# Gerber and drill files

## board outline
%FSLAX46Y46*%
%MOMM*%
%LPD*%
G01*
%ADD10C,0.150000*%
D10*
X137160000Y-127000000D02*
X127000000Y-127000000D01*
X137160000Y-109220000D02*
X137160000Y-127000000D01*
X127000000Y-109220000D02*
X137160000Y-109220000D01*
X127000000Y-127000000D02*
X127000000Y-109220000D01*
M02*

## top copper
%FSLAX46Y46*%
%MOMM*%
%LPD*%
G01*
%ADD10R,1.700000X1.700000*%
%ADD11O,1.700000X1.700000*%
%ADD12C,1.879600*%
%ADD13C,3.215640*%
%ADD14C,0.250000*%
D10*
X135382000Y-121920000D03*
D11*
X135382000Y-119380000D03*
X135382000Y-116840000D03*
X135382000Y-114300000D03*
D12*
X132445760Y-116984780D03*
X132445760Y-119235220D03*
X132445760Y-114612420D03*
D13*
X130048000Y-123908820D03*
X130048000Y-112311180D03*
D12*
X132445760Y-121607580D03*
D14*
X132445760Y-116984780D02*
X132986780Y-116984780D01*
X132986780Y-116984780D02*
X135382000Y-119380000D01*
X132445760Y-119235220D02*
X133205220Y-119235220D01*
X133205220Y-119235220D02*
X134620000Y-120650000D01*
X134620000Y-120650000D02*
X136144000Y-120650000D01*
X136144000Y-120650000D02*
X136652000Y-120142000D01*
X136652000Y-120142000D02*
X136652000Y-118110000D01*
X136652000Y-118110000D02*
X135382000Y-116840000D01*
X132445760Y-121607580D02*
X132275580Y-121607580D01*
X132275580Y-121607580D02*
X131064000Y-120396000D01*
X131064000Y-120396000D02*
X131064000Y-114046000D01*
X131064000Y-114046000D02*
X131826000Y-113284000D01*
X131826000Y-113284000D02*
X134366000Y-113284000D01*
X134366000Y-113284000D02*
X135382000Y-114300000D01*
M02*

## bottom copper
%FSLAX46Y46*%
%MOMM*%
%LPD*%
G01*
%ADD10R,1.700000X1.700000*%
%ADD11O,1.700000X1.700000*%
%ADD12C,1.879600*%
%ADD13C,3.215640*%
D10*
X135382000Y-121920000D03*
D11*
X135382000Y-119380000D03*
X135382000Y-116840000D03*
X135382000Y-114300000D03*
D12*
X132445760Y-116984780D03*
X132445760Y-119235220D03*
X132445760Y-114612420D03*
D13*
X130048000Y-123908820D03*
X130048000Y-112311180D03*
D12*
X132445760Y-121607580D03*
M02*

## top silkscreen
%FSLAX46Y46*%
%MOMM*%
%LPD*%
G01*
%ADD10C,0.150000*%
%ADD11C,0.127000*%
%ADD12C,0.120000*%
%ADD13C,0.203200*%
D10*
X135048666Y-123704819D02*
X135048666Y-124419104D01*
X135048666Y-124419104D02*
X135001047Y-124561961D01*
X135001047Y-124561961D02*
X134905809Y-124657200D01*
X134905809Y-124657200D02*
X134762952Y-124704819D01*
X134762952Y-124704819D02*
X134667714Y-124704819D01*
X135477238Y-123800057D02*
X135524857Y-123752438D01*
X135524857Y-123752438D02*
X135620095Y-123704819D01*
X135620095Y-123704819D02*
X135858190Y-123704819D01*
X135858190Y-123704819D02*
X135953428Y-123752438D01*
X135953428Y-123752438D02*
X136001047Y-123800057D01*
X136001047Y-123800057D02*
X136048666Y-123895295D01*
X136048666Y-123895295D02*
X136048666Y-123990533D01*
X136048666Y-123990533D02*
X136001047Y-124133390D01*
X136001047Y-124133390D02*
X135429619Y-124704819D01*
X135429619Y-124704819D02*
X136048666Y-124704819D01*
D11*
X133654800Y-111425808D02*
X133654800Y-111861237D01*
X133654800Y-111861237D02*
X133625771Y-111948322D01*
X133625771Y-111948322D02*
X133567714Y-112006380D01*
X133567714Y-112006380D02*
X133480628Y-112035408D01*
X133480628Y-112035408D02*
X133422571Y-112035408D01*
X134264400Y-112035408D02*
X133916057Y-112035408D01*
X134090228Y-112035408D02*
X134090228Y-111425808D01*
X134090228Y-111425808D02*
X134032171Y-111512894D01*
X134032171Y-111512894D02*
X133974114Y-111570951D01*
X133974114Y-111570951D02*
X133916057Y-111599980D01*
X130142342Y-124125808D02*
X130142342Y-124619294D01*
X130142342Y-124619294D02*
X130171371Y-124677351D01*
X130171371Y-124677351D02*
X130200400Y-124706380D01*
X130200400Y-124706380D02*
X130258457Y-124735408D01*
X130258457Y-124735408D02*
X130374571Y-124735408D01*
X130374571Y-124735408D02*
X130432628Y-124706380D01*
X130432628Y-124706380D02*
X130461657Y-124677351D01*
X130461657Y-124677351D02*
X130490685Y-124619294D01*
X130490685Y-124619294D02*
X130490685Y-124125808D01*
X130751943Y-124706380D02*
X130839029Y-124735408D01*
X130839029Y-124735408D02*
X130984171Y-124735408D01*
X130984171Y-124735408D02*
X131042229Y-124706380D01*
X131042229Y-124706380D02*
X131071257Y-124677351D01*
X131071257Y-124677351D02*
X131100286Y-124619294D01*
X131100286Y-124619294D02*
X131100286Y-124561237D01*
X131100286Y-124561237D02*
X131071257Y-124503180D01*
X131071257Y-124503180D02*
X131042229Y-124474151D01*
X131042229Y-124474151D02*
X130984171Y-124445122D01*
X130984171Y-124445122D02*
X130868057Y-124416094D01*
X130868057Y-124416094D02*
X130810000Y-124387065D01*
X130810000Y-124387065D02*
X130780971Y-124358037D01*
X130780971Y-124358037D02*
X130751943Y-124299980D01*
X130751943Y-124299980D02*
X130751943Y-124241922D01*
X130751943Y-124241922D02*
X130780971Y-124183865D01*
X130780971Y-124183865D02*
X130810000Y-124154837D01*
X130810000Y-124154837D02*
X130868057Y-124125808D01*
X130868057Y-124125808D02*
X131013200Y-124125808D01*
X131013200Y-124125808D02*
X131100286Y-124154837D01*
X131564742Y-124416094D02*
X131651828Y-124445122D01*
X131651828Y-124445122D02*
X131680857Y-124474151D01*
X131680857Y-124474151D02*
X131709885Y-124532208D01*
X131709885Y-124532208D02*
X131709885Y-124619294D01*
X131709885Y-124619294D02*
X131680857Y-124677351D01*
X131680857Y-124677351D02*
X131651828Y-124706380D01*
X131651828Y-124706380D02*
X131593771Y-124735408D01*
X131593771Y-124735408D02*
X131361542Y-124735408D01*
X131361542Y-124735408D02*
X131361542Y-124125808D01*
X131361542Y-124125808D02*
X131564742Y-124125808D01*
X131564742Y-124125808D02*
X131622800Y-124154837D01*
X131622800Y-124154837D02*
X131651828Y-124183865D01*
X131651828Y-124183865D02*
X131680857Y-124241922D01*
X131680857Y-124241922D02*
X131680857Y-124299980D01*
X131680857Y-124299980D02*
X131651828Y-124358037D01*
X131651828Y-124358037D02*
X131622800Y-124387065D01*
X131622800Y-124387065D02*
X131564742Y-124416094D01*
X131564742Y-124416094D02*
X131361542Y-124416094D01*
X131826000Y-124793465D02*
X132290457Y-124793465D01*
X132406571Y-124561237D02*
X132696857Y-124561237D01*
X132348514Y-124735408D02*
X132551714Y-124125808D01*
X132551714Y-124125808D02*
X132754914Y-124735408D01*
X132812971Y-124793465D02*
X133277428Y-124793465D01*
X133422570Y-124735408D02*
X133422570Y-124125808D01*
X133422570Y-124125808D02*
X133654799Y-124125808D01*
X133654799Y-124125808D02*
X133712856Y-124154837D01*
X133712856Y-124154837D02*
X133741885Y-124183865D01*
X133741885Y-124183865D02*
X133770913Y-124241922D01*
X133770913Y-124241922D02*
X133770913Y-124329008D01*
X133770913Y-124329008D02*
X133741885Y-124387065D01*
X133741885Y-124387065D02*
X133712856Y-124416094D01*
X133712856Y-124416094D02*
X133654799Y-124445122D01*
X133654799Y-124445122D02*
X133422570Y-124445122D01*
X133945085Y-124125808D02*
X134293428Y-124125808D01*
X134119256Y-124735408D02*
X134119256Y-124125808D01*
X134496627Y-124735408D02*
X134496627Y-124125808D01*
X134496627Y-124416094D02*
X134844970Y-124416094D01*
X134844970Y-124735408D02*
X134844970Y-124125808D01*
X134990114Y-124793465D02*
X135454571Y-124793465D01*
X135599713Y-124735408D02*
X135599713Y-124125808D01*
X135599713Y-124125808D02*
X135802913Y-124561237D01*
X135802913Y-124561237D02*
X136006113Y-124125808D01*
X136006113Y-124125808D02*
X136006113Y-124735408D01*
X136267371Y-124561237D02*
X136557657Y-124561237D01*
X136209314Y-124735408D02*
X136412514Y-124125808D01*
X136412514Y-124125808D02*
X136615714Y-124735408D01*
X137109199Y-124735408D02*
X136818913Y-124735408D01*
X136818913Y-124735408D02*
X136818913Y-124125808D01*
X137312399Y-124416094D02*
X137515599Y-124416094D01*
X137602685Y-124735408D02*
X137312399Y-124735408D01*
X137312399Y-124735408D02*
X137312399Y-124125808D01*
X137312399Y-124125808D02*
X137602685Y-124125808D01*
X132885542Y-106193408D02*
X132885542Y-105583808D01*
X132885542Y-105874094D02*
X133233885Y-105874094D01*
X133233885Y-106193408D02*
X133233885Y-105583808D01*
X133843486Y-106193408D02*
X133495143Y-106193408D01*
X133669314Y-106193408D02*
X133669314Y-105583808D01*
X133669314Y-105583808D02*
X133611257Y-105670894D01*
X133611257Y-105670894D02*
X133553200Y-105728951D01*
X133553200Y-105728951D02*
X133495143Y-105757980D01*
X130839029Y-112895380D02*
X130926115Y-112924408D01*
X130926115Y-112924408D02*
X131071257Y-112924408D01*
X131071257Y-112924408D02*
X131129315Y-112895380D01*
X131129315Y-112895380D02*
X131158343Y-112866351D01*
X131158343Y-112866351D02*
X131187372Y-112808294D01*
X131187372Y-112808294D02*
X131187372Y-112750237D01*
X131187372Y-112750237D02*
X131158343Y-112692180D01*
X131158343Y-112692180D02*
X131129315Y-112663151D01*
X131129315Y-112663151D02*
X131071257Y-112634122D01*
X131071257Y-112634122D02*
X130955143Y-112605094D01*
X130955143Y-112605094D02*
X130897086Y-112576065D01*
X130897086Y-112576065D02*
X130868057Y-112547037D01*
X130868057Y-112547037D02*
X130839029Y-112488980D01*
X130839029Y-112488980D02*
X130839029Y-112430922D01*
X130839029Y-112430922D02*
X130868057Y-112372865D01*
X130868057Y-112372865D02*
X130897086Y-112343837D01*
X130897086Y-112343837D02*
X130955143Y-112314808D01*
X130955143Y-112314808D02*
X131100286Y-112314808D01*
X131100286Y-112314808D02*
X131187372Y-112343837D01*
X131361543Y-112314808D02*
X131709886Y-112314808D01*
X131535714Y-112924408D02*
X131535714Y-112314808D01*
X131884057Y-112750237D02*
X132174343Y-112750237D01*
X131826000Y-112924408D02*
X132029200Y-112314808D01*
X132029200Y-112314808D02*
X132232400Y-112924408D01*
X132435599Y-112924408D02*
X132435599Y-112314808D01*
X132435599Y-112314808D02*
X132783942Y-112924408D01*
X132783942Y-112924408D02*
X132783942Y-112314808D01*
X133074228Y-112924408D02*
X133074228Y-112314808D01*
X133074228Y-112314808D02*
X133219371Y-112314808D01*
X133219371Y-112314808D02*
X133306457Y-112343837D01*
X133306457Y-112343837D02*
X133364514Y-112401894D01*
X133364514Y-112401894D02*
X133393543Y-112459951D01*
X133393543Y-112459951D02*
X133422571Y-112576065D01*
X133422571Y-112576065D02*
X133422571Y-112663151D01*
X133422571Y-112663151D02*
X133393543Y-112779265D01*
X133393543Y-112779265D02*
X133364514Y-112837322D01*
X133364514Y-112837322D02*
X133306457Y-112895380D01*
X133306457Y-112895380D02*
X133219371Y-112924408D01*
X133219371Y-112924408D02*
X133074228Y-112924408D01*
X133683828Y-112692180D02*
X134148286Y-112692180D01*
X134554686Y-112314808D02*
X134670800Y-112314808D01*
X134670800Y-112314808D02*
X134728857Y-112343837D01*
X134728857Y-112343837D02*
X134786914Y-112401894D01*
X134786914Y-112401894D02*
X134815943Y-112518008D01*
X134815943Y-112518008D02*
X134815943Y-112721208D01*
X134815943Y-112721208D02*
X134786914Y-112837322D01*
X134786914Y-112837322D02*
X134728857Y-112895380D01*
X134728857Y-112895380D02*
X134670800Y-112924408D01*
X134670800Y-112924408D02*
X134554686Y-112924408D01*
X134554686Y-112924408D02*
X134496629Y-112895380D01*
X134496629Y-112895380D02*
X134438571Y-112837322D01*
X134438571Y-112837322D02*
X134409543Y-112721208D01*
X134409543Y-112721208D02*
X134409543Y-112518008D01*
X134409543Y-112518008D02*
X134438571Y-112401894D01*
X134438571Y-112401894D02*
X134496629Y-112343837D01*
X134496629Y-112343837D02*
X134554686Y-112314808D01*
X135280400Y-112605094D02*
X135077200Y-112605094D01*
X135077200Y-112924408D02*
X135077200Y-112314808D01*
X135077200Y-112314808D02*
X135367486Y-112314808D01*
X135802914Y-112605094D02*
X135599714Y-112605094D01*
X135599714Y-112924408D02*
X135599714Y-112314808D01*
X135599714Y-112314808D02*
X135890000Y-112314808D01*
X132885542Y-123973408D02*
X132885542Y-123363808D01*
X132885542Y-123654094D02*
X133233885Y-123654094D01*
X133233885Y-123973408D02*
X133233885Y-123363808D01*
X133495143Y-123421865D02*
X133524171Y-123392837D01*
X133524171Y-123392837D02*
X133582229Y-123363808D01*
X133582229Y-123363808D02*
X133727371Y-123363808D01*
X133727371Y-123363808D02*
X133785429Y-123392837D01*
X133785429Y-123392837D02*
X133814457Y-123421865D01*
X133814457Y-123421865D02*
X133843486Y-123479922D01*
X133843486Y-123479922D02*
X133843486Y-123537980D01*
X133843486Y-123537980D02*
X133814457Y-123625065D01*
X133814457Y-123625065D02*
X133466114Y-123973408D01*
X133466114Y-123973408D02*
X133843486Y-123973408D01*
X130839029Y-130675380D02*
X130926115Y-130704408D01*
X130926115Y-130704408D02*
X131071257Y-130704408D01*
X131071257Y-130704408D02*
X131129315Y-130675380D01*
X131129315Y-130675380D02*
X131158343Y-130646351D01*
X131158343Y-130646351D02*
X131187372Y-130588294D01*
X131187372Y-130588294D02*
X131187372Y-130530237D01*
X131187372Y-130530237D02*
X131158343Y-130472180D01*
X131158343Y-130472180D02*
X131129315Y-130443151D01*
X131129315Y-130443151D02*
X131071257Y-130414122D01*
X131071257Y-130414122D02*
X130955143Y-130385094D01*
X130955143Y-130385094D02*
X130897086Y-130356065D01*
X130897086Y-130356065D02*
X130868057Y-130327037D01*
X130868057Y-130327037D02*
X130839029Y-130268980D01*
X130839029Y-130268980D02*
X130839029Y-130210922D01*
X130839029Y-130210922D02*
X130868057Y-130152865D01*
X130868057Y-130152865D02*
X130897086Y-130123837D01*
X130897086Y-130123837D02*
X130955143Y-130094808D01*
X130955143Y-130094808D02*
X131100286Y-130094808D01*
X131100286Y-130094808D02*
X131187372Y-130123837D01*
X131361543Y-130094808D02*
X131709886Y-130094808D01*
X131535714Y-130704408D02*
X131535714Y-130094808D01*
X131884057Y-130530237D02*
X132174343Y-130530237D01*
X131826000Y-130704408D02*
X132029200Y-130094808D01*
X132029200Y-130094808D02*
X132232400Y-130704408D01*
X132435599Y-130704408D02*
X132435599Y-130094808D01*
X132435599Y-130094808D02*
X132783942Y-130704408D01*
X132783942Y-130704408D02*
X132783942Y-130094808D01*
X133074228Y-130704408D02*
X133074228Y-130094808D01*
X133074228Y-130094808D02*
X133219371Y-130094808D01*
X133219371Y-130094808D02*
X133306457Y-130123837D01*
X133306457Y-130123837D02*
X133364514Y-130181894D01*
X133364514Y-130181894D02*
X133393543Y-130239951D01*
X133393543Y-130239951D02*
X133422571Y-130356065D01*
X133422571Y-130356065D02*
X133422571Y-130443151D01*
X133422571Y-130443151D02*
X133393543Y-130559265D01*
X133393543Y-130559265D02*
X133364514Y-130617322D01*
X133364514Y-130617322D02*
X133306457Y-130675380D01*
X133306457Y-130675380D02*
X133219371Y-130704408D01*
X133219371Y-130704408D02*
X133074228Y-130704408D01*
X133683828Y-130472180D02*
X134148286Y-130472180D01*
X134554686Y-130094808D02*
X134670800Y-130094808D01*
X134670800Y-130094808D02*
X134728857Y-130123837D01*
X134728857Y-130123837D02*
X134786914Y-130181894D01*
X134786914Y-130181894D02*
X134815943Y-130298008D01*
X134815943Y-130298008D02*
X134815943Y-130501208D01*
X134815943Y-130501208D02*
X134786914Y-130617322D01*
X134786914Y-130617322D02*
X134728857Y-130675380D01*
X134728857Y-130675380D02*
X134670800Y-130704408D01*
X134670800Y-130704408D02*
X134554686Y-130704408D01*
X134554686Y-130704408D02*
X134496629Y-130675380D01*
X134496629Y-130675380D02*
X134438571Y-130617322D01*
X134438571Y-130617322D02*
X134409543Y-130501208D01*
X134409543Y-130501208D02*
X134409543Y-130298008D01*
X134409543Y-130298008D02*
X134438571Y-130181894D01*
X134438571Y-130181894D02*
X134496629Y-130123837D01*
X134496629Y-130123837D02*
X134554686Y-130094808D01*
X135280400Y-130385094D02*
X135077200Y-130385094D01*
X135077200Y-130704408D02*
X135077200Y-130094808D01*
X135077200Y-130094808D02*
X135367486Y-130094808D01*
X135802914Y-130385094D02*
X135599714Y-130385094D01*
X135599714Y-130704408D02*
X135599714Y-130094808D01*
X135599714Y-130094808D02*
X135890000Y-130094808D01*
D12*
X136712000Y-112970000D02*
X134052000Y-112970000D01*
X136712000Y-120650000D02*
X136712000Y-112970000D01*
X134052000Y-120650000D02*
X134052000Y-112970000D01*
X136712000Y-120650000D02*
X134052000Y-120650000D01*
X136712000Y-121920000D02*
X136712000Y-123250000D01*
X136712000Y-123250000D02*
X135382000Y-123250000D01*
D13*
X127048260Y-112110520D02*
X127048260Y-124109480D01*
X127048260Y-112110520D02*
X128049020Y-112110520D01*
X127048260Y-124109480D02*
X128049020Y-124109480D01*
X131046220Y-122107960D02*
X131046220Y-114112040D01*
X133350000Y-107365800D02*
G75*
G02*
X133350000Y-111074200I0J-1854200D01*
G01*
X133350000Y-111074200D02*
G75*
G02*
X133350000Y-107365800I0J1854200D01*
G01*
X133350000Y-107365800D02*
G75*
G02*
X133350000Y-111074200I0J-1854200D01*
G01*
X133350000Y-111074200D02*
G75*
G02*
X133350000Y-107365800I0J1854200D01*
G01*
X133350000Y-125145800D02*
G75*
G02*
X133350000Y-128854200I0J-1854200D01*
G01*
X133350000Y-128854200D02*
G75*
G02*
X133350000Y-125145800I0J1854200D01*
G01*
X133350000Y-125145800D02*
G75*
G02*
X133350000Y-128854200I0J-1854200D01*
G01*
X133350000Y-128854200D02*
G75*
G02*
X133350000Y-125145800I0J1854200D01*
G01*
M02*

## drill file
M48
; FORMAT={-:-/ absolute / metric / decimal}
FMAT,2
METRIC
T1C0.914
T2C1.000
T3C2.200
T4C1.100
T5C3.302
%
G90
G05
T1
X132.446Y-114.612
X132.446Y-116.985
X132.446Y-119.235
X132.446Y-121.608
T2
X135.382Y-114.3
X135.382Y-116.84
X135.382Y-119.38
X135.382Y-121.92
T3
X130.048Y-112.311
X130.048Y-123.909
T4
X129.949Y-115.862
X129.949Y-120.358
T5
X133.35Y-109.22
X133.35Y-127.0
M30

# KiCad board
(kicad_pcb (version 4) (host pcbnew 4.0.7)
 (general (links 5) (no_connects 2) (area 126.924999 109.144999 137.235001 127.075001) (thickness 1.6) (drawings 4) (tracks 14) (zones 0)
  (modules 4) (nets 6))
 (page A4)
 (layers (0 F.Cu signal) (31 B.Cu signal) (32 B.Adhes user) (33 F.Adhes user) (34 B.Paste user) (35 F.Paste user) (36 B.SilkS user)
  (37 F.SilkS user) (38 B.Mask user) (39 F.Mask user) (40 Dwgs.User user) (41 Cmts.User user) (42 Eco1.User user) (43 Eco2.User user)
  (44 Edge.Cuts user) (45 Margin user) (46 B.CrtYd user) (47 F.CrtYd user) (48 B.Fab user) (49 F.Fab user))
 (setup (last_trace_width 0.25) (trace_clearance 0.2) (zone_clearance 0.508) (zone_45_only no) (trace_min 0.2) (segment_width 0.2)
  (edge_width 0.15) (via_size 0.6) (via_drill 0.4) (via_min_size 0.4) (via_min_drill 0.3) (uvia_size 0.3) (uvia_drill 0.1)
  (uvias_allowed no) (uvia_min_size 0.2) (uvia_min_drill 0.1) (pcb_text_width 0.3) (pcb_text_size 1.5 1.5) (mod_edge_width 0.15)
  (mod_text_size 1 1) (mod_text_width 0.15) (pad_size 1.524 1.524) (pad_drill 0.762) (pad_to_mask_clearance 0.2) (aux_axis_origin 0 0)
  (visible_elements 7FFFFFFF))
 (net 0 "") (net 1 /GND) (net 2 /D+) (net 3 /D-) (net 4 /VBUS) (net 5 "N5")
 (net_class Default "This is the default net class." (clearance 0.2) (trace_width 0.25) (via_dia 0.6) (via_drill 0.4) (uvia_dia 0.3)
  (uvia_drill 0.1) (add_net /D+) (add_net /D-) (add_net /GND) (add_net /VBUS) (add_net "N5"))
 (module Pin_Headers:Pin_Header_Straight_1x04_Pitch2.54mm (layer F.Cu) (at 135.382 121.92 180)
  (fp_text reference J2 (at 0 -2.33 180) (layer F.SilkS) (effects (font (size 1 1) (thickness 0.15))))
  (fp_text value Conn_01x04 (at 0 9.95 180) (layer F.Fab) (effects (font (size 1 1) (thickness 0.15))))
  (fp_line (start -1.33 8.95) (end 1.33 8.95) (layer F.SilkS) (width 0.12))
  (fp_line (start -1.33 1.27) (end -1.33 8.95) (layer F.SilkS) (width 0.12))
  (fp_line (start 1.33 1.27) (end 1.33 8.95) (layer F.SilkS) (width 0.12))
  (fp_line (start -1.33 1.27) (end 1.33 1.27) (layer F.SilkS) (width 0.12))
  (fp_line (start -1.33 0) (end -1.33 -1.33) (layer F.SilkS) (width 0.12))
  (fp_line (start -1.33 -1.33) (end 0 -1.33) (layer F.SilkS) (width 0.12))
  (pad 1 thru_hole rect (at 0 0 180) (size 1.7 1.7) (drill 1) (layers *.Cu *.Mask) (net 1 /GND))
  (pad 2 thru_hole oval (at 0 2.54 180) (size 1.7 1.7) (drill 1) (layers *.Cu *.Mask) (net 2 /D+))
  (pad 3 thru_hole oval (at 0 5.08 180) (size 1.7 1.7) (drill 1) (layers *.Cu *.Mask) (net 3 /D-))
  (pad 4 thru_hole oval (at 0 7.62 180) (size 1.7 1.7) (drill 1) (layers *.Cu *.Mask) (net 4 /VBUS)))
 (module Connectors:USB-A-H (layer F.Cu) (at 130.048 118.11)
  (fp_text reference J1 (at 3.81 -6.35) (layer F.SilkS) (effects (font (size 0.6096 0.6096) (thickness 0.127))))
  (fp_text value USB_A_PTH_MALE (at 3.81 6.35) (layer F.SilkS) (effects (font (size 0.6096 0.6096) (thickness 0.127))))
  (fp_line (start -2.99974 -5.99948) (end -2.99974 5.99948) (layer F.SilkS) (width 0.2032))
  (fp_line (start -2.99974 -5.99948) (end -1.99898 -5.99948) (layer F.SilkS) (width 0.2032))
  (fp_line (start -2.99974 5.99948) (end -1.99898 5.99948) (layer F.SilkS) (width 0.2032))
  (fp_line (start 0.99822 3.99796) (end 0.99822 -3.99796) (layer F.SilkS) (width 0.2032))
  (pad D+ thru_hole circle (at 2.39776 -1.12522) (size 1.8796 1.8796) (drill 0.9144) (layers *.Cu *.Mask) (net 2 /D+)
   (solder_mask_margin 0.1016))
  (pad D- thru_hole circle (at 2.39776 1.12522) (size 1.8796 1.8796) (drill 0.9144) (layers *.Cu *.Mask) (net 3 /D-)
   (solder_mask_margin 0.1016))
  (pad GND thru_hole circle (at 2.39776 -3.49758) (size 1.8796 1.8796) (drill 0.9144) (layers *.Cu *.Mask) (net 1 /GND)
   (solder_mask_margin 0.1016))
  (pad SHLD thru_hole circle (at 0 5.79882) (size 3.21564 3.21564) (drill 2.19964) (layers *.Cu *.Mask) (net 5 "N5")
   (solder_mask_margin 0.1016))
  (pad SHLD thru_hole circle (at 0 -5.79882) (size 3.21564 3.21564) (drill 2.19964) (layers *.Cu *.Mask) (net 5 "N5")
   (solder_mask_margin 0.1016))
  (pad VBUS thru_hole circle (at 2.39776 3.49758) (size 1.8796 1.8796) (drill 0.9144) (layers *.Cu *.Mask) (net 4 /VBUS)
   (solder_mask_margin 0.1016))
  (pad "" np_thru_hole circle (at -0.09906 -2.2479) (size 1.09982 1.09982) (drill 1.09982) (layers *.Cu *.Mask) (solder_mask_margin 0.1016))
  (pad "" np_thru_hole circle (at -0.09906 2.2479) (size 1.09982 1.09982) (drill 1.09982) (layers *.Cu *.Mask) (solder_mask_margin 0.1016)))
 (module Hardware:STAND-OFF (layer F.Cu) (at 133.35 109.22)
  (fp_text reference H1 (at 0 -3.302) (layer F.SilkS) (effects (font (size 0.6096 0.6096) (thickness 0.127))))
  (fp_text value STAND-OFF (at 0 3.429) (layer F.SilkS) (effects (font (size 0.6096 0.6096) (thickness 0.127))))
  (fp_arc (start 0 0) (end 0 -1.8542) (angle 180) (layer F.SilkS) (width 0.2032))
  (fp_arc (start 0 0) (end 0 1.8542) (angle 180) (layer F.SilkS) (width 0.2032))
  (fp_arc (start 0 0) (end 0 -1.8542) (angle 180) (layer F.SilkS) (width 0.2032))
  (fp_arc (start 0 0) (end 0 1.8542) (angle 180) (layer F.SilkS) (width 0.2032))
  (pad "" np_thru_hole circle (at 0 0) (size 3.302 3.302) (drill 3.302) (layers *.Cu *.Mask) (solder_mask_margin 0.1016)))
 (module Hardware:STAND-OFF (layer F.Cu) (at 133.35 127)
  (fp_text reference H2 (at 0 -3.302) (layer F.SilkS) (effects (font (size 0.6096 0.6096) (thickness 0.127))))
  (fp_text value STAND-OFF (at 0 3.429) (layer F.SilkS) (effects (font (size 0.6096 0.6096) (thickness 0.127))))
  (fp_arc (start 0 0) (end 0 -1.8542) (angle 180) (layer F.SilkS) (width 0.2032))
  (fp_arc (start 0 0) (end 0 1.8542) (angle 180) (layer F.SilkS) (width 0.2032))
  (fp_arc (start 0 0) (end 0 -1.8542) (angle 180) (layer F.SilkS) (width 0.2032))
  (fp_arc (start 0 0) (end 0 1.8542) (angle 180) (layer F.SilkS) (width 0.2032))
  (pad "" np_thru_hole circle (at 0 0) (size 3.302 3.302) (drill 3.302) (layers *.Cu *.Mask) (solder_mask_margin 0.1016)))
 (gr_line (start 137.16 127) (end 127 127) (angle 90) (layer Edge.Cuts) (width 0.15))
 (gr_line (start 137.16 109.22) (end 137.16 127) (angle 90) (layer Edge.Cuts) (width 0.15))
 (gr_line (start 127 109.22) (end 137.16 109.22) (angle 90) (layer Edge.Cuts) (width 0.15))
 (gr_line (start 127 127) (end 127 109.22) (angle 90) (layer Edge.Cuts) (width 0.15))
 (segment (start 132.44576 116.98478) (end 132.98678 116.98478) (width 0.25) (layer F.Cu) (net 2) (status C00000))
 (segment (start 132.98678 116.98478) (end 135.382 119.38) (width 0.25) (layer F.Cu) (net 2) (status C00000))
 (segment (start 132.44576 119.23522) (end 133.20522 119.23522) (width 0.25) (layer F.Cu) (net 3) (status C00000))
 (segment (start 133.20522 119.23522) (end 134.62 120.65) (width 0.25) (layer F.Cu) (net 3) (status 400000))
 (segment (start 134.62 120.65) (end 136.144 120.65) (width 0.25) (layer F.Cu) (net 3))
 (segment (start 136.144 120.65) (end 136.652 120.142) (width 0.25) (layer F.Cu) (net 3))
 (segment (start 136.652 120.142) (end 136.652 118.11) (width 0.25) (layer F.Cu) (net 3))
 (segment (start 136.652 118.11) (end 135.382 116.84) (width 0.25) (layer F.Cu) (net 3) (status 800000))
 (segment (start 132.44576 121.60758) (end 132.27558 121.60758) (width 0.25) (layer F.Cu) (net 4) (status C00000))
 (segment (start 132.27558 121.60758) (end 131.064 120.396) (width 0.25) (layer F.Cu) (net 4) (status 400000))
 (segment (start 131.064 120.396) (end 131.064 114.046) (width 0.25) (layer F.Cu) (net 4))
 (segment (start 131.064 114.046) (end 131.826 113.284) (width 0.25) (layer F.Cu) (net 4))
 (segment (start 131.826 113.284) (end 134.366 113.284) (width 0.25) (layer F.Cu) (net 4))
 (segment (start 134.366 113.284) (end 135.382 114.3) (width 0.25) (layer F.Cu) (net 4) (status 800000)))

